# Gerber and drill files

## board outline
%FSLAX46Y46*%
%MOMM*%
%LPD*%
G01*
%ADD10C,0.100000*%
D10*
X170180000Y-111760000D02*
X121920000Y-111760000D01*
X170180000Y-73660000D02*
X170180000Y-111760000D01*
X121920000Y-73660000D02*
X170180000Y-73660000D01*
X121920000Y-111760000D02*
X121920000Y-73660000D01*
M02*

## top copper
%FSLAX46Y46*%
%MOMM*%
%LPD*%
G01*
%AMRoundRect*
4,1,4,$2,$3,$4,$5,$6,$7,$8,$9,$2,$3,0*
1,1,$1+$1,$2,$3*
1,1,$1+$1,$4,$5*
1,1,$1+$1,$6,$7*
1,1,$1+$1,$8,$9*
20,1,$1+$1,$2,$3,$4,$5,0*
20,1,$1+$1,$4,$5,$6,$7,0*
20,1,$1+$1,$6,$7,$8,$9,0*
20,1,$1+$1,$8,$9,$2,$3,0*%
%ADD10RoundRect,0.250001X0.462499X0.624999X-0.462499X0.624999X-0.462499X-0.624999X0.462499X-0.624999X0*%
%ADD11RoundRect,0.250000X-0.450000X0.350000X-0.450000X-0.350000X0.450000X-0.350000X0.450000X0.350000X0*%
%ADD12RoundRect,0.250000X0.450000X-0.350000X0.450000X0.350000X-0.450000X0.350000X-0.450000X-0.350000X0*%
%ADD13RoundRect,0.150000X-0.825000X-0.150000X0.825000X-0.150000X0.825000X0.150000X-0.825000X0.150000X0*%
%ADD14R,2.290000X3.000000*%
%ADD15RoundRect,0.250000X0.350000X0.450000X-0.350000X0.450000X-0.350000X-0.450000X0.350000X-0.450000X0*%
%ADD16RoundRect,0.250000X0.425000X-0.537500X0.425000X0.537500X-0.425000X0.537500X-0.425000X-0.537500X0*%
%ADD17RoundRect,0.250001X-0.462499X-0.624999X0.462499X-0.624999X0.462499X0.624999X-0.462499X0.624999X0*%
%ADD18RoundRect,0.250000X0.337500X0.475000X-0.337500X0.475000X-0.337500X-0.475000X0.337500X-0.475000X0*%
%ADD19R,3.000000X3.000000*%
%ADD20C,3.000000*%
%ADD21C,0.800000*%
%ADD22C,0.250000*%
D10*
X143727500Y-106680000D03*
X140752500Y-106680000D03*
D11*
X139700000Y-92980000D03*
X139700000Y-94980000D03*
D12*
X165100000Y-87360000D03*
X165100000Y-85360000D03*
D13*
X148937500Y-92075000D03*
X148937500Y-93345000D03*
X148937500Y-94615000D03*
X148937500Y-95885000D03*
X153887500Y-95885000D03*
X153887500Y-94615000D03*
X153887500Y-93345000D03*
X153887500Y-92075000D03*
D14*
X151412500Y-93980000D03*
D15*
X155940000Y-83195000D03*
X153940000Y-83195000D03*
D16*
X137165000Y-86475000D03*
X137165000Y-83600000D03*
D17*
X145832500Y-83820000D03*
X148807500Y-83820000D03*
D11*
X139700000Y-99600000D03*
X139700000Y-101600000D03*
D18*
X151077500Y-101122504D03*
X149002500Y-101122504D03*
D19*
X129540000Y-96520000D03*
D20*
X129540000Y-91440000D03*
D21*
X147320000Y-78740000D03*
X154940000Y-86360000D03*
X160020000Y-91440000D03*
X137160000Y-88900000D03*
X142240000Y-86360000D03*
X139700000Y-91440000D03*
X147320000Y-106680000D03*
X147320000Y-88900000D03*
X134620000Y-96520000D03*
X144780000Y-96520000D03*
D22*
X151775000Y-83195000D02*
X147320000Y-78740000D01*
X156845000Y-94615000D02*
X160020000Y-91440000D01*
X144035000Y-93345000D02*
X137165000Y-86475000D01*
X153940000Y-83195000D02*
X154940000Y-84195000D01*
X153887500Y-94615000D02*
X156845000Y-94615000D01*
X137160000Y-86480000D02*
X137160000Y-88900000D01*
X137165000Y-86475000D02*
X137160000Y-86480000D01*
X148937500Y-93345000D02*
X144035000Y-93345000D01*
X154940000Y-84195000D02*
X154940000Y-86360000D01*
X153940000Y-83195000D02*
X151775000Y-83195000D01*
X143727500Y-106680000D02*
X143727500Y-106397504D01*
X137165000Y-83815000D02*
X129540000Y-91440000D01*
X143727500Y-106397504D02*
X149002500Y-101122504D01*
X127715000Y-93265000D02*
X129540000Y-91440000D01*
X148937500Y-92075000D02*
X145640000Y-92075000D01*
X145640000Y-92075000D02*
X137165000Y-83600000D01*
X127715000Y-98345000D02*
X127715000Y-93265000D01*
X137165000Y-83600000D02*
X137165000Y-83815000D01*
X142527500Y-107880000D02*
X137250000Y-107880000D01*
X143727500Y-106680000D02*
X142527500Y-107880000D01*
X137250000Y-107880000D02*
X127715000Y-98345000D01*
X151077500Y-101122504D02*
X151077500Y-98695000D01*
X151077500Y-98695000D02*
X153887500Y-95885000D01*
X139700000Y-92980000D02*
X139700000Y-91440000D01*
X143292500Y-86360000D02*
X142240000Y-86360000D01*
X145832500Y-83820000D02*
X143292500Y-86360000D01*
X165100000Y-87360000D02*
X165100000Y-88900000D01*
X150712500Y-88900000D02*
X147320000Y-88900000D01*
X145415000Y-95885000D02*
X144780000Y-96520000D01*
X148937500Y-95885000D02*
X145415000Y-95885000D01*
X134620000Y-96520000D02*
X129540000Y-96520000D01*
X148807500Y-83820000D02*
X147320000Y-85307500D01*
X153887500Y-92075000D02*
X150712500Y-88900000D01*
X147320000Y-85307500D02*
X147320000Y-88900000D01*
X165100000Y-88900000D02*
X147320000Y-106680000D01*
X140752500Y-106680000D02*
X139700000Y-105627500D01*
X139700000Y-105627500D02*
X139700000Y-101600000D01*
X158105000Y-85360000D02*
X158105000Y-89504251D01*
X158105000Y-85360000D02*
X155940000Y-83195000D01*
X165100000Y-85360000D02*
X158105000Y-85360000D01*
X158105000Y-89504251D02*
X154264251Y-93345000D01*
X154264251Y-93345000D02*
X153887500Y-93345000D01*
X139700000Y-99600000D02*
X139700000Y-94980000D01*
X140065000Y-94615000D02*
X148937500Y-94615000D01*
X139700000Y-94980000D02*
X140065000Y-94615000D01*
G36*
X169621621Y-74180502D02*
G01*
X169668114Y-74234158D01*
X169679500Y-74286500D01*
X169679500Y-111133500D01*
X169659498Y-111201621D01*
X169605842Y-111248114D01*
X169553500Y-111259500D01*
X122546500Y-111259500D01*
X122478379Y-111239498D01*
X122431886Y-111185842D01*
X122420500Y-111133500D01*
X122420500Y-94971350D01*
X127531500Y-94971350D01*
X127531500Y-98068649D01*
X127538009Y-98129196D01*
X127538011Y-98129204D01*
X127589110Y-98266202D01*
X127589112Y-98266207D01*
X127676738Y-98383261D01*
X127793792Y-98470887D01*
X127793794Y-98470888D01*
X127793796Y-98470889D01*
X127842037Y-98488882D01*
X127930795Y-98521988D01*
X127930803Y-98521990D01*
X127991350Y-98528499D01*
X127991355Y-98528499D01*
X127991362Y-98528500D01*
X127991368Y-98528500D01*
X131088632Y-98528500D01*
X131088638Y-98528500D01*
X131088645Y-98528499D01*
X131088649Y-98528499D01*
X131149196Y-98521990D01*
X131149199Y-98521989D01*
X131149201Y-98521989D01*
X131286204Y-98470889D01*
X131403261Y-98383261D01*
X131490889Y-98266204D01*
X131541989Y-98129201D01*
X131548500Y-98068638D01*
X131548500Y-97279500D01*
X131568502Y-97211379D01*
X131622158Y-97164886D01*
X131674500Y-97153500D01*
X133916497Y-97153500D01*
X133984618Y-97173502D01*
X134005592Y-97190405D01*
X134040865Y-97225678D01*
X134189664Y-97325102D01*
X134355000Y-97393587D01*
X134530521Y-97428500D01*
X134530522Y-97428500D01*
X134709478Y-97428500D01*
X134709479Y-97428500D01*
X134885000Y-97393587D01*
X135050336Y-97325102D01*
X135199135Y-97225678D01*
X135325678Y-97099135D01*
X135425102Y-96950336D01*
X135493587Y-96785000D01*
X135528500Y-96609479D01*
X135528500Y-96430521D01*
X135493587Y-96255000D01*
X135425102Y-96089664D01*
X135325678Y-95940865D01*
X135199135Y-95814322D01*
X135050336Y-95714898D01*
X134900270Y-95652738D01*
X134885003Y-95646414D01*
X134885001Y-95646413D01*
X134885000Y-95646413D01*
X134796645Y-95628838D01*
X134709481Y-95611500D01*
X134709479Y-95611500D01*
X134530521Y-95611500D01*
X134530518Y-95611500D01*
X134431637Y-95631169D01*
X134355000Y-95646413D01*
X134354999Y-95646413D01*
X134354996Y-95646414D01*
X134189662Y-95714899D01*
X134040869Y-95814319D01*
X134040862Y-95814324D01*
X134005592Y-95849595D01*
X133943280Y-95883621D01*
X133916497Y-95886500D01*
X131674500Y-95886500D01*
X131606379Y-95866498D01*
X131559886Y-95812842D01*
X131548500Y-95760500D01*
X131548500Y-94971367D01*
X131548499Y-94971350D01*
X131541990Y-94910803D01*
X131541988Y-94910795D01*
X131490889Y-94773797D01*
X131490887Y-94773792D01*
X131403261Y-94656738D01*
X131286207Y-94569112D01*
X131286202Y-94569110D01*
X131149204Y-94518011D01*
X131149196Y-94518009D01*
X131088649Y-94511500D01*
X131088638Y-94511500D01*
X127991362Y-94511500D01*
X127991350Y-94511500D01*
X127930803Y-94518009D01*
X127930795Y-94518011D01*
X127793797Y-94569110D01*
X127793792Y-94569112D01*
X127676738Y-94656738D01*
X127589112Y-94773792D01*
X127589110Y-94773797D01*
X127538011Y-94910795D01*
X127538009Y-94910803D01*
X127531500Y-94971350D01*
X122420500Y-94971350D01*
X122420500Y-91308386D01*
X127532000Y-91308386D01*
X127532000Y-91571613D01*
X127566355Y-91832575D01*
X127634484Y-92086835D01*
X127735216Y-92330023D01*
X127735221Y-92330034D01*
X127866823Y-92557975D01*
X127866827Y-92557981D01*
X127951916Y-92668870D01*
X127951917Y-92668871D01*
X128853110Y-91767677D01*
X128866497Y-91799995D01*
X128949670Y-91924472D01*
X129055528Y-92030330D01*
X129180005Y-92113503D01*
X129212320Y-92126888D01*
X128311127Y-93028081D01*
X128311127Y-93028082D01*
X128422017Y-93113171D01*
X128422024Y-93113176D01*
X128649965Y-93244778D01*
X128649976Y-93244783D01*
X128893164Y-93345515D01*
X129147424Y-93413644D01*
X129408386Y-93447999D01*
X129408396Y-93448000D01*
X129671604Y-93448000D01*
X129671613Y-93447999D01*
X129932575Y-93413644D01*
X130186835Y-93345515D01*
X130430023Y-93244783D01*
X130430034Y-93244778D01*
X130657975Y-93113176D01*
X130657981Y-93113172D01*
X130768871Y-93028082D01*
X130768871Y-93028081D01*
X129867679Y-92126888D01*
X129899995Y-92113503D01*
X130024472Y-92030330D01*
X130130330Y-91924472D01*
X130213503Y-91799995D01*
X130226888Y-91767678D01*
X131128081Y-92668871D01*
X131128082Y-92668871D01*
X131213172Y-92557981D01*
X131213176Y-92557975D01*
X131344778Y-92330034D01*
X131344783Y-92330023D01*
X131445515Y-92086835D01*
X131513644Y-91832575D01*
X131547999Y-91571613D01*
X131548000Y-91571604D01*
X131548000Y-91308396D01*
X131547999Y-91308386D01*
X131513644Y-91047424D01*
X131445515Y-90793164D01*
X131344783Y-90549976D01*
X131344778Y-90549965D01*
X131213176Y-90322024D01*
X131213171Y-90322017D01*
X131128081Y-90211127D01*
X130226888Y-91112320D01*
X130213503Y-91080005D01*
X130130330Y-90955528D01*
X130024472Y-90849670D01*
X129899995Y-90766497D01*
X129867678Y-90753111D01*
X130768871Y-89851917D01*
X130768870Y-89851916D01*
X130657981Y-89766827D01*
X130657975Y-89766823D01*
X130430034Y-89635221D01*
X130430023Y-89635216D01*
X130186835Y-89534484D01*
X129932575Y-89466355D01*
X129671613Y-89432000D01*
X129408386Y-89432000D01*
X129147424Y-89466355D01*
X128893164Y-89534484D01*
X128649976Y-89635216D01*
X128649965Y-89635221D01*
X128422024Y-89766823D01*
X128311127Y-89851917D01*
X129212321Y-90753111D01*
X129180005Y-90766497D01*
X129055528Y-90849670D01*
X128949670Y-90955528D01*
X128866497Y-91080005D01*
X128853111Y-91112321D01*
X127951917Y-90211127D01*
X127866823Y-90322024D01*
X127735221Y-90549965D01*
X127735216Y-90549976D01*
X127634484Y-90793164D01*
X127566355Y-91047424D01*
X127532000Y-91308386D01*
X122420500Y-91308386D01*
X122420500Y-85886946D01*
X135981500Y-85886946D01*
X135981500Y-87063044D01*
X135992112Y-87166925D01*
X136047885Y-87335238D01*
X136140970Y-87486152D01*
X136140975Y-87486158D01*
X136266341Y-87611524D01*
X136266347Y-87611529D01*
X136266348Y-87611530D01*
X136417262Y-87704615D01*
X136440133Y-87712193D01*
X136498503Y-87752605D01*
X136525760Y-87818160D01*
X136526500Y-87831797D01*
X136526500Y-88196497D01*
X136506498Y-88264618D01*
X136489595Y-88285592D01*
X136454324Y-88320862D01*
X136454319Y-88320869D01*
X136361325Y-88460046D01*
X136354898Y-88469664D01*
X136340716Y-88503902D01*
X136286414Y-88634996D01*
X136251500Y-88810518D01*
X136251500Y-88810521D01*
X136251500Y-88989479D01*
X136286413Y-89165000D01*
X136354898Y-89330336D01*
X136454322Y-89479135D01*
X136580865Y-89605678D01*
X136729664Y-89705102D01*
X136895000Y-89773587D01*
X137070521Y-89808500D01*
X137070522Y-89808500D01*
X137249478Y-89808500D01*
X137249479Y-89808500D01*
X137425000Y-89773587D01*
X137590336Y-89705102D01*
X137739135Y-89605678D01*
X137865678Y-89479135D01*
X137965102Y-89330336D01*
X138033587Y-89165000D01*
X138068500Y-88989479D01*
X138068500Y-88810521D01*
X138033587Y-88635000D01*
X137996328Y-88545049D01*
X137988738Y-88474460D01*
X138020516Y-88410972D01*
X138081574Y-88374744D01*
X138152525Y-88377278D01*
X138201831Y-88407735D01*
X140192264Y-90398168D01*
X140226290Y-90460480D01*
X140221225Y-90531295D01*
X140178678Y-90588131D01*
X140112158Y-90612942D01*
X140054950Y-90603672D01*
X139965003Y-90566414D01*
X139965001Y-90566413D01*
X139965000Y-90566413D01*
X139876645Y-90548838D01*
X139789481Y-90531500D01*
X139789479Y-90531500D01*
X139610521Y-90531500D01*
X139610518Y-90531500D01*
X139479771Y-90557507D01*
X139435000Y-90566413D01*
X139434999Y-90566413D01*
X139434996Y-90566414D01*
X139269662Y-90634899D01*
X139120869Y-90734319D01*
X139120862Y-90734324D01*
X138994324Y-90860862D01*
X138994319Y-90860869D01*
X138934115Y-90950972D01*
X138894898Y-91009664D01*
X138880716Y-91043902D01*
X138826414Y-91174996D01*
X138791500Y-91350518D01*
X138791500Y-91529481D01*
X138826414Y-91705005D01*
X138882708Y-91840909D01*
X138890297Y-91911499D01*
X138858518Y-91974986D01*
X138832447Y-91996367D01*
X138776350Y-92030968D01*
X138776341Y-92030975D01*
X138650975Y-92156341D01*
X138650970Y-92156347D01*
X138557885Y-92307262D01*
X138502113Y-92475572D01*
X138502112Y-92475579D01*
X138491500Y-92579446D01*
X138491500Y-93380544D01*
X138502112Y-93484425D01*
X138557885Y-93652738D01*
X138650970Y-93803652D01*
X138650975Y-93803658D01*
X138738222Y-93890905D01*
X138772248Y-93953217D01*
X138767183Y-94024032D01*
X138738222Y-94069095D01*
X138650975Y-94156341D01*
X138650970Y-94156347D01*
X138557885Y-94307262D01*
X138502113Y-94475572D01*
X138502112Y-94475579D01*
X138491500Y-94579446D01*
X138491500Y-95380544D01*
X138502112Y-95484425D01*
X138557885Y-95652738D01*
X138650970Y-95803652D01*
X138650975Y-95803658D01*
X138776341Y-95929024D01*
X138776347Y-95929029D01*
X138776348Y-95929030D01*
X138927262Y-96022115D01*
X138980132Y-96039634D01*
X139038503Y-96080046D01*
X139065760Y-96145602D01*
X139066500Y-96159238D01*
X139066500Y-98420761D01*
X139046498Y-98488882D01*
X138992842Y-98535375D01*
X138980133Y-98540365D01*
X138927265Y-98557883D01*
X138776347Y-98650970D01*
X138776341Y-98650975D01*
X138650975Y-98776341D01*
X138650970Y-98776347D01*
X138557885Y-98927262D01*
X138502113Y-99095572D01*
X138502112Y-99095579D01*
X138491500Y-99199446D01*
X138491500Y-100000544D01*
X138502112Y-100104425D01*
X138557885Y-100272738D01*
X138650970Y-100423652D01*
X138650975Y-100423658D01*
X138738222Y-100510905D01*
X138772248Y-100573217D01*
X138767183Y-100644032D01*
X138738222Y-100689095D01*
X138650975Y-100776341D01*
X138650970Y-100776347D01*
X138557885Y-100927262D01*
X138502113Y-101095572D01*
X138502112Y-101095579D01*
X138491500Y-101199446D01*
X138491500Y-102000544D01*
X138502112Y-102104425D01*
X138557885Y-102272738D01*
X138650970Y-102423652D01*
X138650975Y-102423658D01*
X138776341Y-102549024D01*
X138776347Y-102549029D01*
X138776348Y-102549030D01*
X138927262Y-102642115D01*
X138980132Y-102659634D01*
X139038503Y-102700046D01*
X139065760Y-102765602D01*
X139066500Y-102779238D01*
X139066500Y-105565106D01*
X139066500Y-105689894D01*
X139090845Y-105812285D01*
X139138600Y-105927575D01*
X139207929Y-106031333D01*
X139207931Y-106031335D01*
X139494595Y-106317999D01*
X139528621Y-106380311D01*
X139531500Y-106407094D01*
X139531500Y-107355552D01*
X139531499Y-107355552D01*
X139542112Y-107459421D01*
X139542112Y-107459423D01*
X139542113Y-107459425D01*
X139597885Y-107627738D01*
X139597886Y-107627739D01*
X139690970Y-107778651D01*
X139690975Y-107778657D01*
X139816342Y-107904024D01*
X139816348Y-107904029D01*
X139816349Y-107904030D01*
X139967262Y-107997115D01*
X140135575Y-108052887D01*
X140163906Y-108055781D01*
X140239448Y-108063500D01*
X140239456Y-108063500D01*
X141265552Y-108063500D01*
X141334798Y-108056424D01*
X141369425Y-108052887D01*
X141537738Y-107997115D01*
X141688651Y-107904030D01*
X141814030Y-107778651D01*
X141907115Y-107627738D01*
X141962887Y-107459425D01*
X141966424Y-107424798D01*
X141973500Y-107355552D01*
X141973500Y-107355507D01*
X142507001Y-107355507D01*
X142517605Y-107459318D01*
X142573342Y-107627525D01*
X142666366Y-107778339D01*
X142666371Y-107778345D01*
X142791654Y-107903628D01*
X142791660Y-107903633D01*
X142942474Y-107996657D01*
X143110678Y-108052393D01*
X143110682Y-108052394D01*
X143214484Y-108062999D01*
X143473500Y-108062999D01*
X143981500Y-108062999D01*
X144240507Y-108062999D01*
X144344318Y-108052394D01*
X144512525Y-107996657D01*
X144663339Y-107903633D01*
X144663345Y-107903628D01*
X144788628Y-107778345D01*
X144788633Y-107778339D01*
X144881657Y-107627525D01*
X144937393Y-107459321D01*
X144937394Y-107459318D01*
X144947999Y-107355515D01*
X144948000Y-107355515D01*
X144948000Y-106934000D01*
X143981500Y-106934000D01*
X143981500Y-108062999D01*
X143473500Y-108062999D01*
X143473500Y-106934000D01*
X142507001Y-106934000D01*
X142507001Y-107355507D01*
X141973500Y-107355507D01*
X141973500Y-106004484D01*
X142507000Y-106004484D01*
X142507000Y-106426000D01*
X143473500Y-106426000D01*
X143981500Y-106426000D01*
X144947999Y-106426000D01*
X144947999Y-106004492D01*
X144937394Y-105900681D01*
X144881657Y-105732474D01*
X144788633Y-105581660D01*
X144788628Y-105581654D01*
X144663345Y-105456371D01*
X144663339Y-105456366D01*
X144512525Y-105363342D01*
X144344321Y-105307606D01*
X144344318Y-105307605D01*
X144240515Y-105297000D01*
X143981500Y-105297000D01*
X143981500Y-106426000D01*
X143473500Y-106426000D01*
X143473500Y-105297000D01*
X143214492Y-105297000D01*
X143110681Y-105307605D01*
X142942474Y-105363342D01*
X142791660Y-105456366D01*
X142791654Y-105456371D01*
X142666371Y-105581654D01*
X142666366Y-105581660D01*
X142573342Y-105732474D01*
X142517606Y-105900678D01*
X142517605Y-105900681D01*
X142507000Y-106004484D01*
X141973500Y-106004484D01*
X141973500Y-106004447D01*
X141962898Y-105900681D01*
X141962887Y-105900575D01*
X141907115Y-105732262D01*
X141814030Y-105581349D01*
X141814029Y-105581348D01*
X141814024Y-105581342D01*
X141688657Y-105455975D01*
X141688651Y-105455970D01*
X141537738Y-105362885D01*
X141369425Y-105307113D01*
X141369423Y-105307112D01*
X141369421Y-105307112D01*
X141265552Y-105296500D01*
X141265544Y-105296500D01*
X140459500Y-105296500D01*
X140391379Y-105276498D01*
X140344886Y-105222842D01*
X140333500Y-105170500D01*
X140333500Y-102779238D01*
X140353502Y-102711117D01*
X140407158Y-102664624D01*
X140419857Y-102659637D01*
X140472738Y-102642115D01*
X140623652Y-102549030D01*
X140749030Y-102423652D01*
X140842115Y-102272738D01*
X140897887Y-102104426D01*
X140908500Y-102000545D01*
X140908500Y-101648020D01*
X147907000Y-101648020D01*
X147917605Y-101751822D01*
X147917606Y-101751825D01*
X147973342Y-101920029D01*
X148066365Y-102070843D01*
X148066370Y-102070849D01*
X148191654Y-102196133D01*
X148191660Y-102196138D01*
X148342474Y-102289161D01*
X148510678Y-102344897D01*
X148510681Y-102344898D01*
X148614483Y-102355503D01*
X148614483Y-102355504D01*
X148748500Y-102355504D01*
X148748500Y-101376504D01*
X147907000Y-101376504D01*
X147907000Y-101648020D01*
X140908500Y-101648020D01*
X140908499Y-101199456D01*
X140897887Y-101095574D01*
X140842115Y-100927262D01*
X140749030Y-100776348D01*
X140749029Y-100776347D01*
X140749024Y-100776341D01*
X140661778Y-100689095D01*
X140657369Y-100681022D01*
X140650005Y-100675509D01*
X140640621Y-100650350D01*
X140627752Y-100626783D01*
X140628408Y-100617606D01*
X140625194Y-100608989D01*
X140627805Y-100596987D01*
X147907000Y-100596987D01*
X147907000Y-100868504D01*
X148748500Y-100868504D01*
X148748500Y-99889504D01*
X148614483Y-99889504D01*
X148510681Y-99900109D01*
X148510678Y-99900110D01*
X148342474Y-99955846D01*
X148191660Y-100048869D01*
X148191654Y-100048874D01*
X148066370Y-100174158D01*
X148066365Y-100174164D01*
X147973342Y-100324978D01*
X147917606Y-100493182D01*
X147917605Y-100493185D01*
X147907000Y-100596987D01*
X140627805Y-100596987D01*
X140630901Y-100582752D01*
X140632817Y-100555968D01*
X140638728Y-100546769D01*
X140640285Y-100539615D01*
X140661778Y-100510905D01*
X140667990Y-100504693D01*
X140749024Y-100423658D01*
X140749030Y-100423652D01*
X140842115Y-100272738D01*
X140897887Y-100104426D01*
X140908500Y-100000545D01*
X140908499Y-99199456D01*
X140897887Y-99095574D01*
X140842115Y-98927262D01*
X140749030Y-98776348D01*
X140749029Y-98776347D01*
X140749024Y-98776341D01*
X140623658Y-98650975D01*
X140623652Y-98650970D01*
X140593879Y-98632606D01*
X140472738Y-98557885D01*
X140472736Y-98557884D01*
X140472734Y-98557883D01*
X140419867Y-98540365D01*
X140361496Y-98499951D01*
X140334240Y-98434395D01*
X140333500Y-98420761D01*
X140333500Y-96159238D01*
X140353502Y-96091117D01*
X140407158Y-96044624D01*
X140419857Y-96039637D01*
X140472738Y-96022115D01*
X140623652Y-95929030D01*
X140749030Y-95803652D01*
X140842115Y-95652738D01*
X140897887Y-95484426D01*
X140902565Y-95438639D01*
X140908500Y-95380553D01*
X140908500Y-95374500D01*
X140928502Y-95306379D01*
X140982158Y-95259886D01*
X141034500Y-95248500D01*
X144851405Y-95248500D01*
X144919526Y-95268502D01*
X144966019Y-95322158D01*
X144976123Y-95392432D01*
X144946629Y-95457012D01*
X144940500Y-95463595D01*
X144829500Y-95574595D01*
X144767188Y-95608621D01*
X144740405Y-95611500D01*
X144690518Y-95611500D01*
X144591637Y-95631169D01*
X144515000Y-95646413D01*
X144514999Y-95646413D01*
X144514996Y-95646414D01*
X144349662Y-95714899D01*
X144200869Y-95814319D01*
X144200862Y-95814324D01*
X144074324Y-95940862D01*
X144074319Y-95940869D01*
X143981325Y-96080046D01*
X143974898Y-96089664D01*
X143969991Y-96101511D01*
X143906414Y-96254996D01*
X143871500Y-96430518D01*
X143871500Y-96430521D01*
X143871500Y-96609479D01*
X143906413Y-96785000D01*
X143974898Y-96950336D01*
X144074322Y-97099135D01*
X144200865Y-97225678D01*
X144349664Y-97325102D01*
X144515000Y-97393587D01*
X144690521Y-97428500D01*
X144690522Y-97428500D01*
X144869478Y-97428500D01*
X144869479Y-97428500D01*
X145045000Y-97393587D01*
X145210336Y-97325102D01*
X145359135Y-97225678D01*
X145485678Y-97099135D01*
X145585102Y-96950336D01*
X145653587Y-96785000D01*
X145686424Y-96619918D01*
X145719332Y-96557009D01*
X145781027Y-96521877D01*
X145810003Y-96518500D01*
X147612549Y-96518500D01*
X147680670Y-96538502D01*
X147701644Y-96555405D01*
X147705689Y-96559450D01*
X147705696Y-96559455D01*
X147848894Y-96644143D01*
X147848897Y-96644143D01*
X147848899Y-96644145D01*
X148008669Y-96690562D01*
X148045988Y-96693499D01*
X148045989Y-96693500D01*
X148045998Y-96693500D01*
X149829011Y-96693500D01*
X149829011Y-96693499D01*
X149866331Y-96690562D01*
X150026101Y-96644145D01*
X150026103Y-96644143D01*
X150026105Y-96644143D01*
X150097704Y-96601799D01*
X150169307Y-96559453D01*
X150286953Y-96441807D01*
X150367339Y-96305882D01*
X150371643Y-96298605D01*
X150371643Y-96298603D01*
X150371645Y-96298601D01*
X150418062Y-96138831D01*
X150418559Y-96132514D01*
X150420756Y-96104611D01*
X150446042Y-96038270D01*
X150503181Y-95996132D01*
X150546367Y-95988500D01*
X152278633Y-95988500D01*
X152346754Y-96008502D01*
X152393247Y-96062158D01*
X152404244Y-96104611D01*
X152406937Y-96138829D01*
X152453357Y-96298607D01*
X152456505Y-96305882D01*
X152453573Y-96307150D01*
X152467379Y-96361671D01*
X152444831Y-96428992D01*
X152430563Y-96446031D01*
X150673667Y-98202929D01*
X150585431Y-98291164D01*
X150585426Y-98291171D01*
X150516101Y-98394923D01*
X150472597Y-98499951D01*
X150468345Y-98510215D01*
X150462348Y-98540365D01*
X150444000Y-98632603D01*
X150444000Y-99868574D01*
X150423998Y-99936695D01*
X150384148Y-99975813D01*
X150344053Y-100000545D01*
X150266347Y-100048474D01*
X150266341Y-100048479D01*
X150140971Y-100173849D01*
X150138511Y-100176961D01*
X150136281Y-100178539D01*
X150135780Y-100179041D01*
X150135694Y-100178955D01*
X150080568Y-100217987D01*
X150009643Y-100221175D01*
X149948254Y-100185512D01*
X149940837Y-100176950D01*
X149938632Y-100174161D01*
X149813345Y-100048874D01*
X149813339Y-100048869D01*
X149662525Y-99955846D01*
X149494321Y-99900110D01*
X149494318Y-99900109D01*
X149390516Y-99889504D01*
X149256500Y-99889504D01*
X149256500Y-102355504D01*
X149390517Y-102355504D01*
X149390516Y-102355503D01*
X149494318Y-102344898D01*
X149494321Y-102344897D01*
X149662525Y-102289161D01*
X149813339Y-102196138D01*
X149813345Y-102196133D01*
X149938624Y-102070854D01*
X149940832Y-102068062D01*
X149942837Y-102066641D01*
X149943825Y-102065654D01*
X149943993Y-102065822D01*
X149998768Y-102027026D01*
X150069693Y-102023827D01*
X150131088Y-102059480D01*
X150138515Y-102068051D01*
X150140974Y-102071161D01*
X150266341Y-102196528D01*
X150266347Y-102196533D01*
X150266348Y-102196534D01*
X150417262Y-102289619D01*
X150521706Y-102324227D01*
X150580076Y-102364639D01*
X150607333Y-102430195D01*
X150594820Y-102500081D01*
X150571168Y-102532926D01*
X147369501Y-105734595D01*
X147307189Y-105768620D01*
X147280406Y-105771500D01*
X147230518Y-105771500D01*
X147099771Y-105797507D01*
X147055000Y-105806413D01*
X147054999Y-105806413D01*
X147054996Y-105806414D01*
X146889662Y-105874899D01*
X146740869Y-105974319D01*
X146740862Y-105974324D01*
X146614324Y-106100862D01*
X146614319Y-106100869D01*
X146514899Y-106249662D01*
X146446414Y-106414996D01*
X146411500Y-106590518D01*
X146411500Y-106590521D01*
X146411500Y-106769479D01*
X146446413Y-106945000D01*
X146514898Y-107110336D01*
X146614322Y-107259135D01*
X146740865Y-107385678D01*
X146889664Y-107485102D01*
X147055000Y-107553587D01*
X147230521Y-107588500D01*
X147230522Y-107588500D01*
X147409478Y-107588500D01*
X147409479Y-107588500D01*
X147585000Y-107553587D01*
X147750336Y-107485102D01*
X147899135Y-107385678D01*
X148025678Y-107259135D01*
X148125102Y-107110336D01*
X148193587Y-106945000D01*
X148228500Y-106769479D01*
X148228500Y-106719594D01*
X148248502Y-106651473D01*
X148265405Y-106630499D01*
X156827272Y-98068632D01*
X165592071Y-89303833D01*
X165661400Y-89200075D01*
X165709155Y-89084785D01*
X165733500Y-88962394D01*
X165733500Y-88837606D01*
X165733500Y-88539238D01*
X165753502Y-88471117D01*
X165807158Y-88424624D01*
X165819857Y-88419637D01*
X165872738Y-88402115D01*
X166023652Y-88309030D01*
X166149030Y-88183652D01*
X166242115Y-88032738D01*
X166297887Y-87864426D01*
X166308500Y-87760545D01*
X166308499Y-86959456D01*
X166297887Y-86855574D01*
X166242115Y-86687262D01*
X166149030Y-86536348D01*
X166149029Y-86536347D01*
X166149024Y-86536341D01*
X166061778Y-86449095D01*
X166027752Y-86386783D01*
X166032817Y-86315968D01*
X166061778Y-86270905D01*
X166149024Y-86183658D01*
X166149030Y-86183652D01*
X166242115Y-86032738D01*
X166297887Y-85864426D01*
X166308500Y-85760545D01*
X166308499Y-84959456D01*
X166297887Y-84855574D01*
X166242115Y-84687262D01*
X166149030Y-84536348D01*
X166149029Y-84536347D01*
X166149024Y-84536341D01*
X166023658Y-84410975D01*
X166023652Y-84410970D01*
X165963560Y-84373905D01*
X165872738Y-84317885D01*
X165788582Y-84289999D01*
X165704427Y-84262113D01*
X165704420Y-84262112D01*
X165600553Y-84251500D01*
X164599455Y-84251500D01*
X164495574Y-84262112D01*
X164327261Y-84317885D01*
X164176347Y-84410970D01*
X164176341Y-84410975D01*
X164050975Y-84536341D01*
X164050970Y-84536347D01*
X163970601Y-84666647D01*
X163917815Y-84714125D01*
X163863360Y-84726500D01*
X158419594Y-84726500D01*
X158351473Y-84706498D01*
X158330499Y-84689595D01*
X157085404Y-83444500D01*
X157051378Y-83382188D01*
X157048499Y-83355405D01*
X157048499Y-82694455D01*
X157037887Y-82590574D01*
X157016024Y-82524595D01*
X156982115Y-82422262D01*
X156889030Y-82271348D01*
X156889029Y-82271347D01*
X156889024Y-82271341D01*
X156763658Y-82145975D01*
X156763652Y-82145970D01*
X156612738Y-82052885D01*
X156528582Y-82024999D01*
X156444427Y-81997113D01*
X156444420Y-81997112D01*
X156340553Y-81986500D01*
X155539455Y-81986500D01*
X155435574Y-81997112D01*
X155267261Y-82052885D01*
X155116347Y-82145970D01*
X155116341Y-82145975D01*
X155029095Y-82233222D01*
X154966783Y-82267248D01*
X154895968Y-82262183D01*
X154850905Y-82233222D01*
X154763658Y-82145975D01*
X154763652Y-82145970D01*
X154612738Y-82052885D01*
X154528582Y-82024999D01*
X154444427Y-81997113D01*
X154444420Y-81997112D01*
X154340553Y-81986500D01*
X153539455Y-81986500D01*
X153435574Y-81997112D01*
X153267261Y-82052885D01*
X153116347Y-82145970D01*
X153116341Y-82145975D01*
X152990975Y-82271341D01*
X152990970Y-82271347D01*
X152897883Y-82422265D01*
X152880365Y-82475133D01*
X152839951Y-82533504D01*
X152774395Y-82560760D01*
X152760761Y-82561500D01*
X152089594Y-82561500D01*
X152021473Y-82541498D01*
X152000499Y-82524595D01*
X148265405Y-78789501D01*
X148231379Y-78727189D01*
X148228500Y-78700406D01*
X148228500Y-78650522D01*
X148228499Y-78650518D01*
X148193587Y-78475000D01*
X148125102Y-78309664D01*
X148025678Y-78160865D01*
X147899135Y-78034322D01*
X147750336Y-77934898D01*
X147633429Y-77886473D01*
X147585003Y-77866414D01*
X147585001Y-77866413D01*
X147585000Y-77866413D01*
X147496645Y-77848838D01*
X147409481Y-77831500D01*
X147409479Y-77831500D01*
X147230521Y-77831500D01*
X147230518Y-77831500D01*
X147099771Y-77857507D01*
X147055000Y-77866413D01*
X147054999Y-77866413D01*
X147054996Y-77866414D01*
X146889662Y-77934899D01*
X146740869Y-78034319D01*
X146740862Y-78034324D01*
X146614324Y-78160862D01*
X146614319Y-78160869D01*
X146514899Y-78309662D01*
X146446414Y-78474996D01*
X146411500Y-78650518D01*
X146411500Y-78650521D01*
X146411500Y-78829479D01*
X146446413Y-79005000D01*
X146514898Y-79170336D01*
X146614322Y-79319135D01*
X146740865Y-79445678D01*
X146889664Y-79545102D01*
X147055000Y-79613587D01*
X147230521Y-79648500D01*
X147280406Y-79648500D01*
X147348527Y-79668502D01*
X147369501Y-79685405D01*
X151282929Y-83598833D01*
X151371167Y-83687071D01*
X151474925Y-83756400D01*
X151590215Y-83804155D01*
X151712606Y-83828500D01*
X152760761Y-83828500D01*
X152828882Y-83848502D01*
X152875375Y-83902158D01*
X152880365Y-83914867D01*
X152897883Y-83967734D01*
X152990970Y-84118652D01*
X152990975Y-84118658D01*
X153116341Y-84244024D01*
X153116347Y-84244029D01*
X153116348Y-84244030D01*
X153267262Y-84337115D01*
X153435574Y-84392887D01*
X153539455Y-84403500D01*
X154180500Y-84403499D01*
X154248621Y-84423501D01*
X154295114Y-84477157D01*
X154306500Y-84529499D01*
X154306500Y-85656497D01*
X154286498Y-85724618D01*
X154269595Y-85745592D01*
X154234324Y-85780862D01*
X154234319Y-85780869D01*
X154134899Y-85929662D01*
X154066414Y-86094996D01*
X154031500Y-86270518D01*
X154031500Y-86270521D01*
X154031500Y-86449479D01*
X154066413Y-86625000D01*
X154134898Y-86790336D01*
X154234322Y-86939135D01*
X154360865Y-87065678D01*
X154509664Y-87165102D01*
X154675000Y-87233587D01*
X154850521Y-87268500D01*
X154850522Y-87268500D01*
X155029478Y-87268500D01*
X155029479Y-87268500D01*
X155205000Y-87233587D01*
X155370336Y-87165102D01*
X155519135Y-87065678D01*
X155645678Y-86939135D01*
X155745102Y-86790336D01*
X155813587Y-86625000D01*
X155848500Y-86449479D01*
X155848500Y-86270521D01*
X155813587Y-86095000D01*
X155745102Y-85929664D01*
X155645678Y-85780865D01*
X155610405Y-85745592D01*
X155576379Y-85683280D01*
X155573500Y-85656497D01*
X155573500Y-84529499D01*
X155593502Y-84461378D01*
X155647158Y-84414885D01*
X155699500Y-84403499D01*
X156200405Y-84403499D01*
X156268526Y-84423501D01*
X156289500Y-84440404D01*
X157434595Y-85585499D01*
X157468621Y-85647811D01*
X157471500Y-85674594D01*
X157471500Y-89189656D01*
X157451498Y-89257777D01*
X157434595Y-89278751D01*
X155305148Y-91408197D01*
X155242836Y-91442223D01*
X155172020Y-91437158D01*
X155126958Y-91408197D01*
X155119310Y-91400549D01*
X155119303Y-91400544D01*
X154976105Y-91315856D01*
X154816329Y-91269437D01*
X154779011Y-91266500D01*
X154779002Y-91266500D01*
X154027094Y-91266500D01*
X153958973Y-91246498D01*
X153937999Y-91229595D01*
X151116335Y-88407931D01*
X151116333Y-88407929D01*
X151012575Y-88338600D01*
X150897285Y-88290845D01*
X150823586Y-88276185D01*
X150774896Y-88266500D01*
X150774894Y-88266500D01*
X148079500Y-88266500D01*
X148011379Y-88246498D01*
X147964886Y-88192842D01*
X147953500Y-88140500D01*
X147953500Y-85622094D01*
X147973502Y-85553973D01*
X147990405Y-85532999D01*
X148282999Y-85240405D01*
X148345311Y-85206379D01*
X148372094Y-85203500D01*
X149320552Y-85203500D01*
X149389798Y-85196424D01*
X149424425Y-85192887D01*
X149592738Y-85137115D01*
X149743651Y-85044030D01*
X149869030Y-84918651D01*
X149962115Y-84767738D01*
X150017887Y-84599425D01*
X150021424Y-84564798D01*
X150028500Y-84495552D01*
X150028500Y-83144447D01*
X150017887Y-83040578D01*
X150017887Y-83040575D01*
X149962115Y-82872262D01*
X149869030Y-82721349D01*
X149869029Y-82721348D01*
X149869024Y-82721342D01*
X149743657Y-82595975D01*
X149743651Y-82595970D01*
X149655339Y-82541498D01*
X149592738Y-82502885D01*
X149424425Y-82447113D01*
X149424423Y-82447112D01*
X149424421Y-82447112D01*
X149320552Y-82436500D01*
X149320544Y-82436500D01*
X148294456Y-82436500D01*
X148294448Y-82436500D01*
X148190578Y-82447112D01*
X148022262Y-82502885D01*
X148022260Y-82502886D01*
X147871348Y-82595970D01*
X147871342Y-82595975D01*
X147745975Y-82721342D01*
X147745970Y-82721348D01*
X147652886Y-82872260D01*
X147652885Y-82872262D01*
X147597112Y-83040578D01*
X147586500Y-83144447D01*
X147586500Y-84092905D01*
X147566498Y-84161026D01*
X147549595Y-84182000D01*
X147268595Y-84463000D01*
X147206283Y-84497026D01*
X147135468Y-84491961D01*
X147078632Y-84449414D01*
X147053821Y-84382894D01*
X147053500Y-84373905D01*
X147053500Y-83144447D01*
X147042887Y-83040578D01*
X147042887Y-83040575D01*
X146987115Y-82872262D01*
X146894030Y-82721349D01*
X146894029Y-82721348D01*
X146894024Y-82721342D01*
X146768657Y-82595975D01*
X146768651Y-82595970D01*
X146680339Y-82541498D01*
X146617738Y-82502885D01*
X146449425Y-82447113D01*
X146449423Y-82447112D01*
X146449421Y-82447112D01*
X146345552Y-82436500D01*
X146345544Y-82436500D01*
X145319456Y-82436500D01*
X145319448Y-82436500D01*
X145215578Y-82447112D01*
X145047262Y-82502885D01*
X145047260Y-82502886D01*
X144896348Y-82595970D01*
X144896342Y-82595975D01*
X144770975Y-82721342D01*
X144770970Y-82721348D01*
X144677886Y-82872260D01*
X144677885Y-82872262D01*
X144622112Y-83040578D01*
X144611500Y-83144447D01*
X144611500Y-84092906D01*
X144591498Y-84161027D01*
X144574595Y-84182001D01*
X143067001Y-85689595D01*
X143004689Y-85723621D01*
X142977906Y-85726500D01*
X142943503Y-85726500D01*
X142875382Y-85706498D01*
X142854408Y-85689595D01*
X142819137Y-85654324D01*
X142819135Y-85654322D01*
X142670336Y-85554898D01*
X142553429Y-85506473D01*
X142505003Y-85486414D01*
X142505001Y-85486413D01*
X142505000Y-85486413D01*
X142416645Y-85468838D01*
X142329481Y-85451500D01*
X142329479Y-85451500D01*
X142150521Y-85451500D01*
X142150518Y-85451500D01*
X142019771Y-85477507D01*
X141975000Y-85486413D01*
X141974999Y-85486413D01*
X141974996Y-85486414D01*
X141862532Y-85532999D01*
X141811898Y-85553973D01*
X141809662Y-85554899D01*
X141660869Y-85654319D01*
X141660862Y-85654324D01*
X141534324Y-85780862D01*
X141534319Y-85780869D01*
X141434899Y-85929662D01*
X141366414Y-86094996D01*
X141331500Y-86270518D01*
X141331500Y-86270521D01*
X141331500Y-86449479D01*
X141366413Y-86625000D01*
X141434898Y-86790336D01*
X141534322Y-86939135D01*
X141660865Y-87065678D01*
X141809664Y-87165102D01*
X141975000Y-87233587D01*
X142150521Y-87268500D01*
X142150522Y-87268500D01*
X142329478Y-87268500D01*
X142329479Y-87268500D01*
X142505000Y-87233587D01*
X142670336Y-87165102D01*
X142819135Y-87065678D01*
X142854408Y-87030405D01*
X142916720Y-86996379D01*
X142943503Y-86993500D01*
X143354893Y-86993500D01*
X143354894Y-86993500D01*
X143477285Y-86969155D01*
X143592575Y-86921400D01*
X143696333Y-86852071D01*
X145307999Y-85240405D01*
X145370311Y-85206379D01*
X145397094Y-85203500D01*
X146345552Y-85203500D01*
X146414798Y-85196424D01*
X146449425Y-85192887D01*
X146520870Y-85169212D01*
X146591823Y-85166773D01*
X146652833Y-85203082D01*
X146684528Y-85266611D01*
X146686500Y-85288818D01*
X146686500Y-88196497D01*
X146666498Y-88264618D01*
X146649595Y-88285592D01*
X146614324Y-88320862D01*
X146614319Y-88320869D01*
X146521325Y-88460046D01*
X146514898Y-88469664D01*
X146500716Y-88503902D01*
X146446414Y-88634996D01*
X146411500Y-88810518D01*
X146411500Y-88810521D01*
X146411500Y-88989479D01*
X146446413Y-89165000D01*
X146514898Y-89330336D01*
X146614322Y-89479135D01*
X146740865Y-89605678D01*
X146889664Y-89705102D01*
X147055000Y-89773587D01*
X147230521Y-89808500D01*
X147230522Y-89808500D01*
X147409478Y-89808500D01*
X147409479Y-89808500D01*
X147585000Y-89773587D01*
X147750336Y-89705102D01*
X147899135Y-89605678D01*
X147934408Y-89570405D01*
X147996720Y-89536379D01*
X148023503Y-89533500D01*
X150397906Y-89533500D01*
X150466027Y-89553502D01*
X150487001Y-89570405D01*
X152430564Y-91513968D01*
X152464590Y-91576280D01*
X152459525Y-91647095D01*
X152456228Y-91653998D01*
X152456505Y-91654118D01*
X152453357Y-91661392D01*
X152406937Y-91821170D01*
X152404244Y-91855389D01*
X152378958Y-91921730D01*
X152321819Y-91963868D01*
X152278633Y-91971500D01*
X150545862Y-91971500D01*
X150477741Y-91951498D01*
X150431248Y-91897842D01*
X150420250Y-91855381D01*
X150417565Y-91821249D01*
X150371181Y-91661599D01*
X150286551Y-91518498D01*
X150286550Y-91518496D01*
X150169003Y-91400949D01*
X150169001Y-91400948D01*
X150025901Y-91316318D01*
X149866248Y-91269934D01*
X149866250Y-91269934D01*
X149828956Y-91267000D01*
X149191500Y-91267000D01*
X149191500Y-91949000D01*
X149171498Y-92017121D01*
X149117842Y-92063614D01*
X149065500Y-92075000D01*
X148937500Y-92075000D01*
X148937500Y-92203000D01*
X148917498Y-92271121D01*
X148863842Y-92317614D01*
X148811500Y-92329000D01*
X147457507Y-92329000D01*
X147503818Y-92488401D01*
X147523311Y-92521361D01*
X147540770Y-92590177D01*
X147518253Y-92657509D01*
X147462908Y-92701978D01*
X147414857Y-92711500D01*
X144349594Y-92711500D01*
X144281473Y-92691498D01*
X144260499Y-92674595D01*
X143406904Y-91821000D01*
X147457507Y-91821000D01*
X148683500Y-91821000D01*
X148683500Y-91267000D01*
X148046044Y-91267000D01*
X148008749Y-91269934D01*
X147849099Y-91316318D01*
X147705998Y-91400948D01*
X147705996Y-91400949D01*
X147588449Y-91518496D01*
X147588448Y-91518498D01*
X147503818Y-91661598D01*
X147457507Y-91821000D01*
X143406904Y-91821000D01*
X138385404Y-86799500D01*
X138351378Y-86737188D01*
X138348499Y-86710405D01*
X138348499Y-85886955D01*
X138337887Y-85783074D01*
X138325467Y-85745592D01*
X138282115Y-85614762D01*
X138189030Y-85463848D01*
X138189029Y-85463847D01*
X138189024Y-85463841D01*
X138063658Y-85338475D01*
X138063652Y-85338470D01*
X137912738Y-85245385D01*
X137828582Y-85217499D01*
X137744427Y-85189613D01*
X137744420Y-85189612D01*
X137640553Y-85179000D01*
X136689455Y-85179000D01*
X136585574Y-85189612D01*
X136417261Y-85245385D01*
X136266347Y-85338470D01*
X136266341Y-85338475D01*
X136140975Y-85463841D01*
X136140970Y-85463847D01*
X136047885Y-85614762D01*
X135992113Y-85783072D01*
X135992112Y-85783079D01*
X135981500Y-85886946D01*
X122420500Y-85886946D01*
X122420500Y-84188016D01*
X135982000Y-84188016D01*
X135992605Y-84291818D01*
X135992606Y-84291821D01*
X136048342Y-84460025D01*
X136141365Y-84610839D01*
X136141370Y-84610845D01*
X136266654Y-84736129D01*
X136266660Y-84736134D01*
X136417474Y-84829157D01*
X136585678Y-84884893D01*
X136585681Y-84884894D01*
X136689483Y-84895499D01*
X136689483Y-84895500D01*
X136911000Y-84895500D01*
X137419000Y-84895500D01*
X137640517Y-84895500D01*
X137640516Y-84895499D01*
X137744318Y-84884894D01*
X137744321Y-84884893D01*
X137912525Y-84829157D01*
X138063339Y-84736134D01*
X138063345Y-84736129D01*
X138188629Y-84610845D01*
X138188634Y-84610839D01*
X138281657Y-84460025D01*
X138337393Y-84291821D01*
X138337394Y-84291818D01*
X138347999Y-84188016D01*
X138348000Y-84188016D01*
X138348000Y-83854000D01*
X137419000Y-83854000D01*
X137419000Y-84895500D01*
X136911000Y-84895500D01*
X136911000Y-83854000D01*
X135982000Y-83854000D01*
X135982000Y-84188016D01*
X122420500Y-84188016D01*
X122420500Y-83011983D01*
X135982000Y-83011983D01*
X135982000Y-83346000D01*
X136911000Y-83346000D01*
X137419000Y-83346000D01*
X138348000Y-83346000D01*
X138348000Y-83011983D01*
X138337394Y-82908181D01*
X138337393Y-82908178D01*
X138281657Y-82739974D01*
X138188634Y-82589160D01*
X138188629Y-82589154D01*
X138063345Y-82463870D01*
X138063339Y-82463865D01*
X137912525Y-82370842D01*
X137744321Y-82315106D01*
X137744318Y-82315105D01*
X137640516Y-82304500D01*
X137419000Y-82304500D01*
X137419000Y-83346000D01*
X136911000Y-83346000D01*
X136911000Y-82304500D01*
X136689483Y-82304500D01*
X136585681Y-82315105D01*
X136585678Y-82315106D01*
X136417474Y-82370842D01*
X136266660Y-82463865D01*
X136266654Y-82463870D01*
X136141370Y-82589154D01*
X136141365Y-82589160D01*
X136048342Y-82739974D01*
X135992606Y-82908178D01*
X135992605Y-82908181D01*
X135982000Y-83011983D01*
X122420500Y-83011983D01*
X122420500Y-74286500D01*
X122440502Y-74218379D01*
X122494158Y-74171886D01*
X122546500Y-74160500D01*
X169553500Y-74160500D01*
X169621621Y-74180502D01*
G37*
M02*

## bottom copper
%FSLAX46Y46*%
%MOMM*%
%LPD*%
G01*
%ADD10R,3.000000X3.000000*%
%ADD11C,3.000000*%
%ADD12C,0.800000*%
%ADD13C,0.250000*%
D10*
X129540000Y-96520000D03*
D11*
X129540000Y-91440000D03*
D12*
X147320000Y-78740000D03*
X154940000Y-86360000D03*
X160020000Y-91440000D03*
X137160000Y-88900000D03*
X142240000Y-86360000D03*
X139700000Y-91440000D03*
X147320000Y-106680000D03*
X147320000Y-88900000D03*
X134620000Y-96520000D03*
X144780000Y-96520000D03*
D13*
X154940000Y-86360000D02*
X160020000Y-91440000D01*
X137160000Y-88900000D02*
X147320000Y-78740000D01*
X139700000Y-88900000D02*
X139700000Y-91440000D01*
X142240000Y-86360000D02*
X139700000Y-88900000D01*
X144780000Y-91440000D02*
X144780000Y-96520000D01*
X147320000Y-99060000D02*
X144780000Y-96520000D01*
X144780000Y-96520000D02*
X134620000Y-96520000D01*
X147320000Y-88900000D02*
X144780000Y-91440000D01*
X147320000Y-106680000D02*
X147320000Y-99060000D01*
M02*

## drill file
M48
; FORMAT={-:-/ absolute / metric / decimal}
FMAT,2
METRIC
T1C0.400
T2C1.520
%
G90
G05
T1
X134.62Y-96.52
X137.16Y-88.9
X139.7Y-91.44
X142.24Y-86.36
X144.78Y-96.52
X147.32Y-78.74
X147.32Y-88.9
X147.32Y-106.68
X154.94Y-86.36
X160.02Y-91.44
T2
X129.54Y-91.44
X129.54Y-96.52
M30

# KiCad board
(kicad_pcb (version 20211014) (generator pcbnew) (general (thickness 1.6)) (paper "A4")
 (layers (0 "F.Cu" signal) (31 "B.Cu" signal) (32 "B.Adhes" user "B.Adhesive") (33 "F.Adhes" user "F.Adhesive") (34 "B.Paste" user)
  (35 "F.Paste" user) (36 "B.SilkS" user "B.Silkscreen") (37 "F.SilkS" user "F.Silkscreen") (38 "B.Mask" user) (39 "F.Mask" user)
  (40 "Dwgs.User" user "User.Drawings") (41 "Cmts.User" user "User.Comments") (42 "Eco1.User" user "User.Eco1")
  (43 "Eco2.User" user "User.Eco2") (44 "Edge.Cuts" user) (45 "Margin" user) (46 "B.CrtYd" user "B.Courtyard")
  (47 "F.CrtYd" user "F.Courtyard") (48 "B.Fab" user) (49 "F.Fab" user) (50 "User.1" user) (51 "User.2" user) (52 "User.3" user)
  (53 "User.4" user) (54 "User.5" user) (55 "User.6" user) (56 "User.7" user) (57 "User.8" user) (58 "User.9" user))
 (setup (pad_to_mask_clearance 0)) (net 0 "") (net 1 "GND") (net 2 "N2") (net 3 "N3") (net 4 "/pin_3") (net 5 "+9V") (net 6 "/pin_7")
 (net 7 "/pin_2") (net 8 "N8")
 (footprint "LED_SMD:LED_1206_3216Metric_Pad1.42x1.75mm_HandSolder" (layer "F.Cu") (at 142.24 106.68 180)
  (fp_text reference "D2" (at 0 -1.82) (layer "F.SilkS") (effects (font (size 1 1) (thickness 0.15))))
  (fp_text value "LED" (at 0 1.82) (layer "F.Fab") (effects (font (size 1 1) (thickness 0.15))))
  (pad "1" smd roundrect (at -1.4875 0 180) (size 1.425 1.75) (layers "F.Cu" "F.Paste" "F.Mask") (roundrect_rratio 0.1754392982)
   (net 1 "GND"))
  (pad "2" smd roundrect (at 1.4875 0 180) (size 1.425 1.75) (layers "F.Cu" "F.Paste" "F.Mask") (roundrect_rratio 0.1754392982) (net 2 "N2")))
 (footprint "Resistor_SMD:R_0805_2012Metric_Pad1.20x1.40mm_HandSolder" (layer "F.Cu") (at 139.7 93.98 -90)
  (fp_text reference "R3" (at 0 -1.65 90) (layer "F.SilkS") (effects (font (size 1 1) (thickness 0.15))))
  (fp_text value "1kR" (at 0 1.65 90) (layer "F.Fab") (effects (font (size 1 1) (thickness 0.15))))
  (pad "1" smd roundrect (at -1 0 270) (size 1.2 1.4) (layers "F.Cu" "F.Paste" "F.Mask") (roundrect_rratio 0.2083333333) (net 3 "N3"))
  (pad "2" smd roundrect (at 1 0 270) (size 1.2 1.4) (layers "F.Cu" "F.Paste" "F.Mask") (roundrect_rratio 0.2083333333) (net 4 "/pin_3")))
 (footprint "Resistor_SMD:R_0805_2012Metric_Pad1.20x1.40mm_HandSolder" (layer "F.Cu") (at 165.1 86.36 90)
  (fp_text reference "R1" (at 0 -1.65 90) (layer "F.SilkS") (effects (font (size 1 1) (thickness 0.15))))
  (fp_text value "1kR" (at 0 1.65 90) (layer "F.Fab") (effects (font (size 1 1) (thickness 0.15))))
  (pad "1" smd roundrect (at -1 0 90) (size 1.2 1.4) (layers "F.Cu" "F.Paste" "F.Mask") (roundrect_rratio 0.2083333333) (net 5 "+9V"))
  (pad "2" smd roundrect (at 1 0 90) (size 1.2 1.4) (layers "F.Cu" "F.Paste" "F.Mask") (roundrect_rratio 0.2083333333) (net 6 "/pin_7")))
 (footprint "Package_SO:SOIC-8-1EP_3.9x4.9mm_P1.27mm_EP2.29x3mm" (layer "F.Cu") (at 151.4125 93.98)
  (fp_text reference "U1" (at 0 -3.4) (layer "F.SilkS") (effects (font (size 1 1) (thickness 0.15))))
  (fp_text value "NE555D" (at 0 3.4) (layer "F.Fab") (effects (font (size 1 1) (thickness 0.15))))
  (pad "" smd roundrect (at 0.57 0.75) (size 0.92 1.21) (layers "F.Paste") (roundrect_rratio 0.25))
  (pad "" smd roundrect (at 0.57 -0.75) (size 0.92 1.21) (layers "F.Paste") (roundrect_rratio 0.25))
  (pad "" smd roundrect (at -0.57 -0.75) (size 0.92 1.21) (layers "F.Paste") (roundrect_rratio 0.25))
  (pad "" smd roundrect (at -0.57 0.75) (size 0.92 1.21) (layers "F.Paste") (roundrect_rratio 0.25))
  (pad "1" smd roundrect (at -2.475 -1.905) (size 1.95 0.6) (layers "F.Cu" "F.Paste" "F.Mask") (roundrect_rratio 0.25) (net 1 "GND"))
  (pad "2" smd roundrect (at -2.475 -0.635) (size 1.95 0.6) (layers "F.Cu" "F.Paste" "F.Mask") (roundrect_rratio 0.25) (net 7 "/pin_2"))
  (pad "3" smd roundrect (at -2.475 0.635) (size 1.95 0.6) (layers "F.Cu" "F.Paste" "F.Mask") (roundrect_rratio 0.25) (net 4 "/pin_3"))
  (pad "4" smd roundrect (at -2.475 1.905) (size 1.95 0.6) (layers "F.Cu" "F.Paste" "F.Mask") (roundrect_rratio 0.25) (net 5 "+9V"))
  (pad "5" smd roundrect (at 2.475 1.905) (size 1.95 0.6) (layers "F.Cu" "F.Paste" "F.Mask") (roundrect_rratio 0.25) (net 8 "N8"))
  (pad "6" smd roundrect (at 2.475 0.635) (size 1.95 0.6) (layers "F.Cu" "F.Paste" "F.Mask") (roundrect_rratio 0.25) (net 7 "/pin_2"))
  (pad "7" smd roundrect (at 2.475 -0.635) (size 1.95 0.6) (layers "F.Cu" "F.Paste" "F.Mask") (roundrect_rratio 0.25) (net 6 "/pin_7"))
  (pad "8" smd roundrect (at 2.475 -1.905) (size 1.95 0.6) (layers "F.Cu" "F.Paste" "F.Mask") (roundrect_rratio 0.25) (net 5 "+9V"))
  (pad "9" smd rect (at 0 0) (size 2.29 3) (layers "F.Cu" "F.Mask")))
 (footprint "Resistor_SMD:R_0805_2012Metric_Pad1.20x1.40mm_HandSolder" (layer "F.Cu") (at 154.94 83.195 180)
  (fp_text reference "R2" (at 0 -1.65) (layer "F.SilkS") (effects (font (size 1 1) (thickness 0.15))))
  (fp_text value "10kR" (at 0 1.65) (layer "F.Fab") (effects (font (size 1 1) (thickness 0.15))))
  (pad "1" smd roundrect (at -1 0 180) (size 1.2 1.4) (layers "F.Cu" "F.Paste" "F.Mask") (roundrect_rratio 0.2083333333) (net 6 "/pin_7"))
  (pad "2" smd roundrect (at 1 0 180) (size 1.2 1.4) (layers "F.Cu" "F.Paste" "F.Mask") (roundrect_rratio 0.2083333333) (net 7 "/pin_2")))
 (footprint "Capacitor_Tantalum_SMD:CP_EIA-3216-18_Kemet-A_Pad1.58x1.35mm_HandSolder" (layer "F.Cu") (at 137.165 85.0375 90)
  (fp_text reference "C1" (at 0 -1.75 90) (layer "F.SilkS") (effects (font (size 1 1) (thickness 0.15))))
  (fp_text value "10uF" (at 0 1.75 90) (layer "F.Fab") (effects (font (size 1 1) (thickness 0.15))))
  (pad "1" smd roundrect (at -1.4375 0 90) (size 1.575 1.35) (layers "F.Cu" "F.Paste" "F.Mask") (roundrect_rratio 0.1851851852)
   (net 7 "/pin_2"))
  (pad "2" smd roundrect (at 1.4375 0 90) (size 1.575 1.35) (layers "F.Cu" "F.Paste" "F.Mask") (roundrect_rratio 0.1851851852) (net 1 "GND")))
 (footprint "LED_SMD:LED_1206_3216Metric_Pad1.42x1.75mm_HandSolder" (layer "F.Cu") (at 147.32 83.82)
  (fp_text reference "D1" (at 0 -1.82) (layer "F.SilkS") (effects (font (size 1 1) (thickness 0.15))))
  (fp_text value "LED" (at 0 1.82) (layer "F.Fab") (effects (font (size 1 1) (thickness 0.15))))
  (pad "1" smd roundrect (at -1.4875 0) (size 1.425 1.75) (layers "F.Cu" "F.Paste" "F.Mask") (roundrect_rratio 0.1754392982) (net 3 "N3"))
  (pad "2" smd roundrect (at 1.4875 0) (size 1.425 1.75) (layers "F.Cu" "F.Paste" "F.Mask") (roundrect_rratio 0.1754392982) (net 5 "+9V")))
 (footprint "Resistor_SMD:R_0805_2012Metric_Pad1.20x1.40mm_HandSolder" (layer "F.Cu") (at 139.7 100.6 -90)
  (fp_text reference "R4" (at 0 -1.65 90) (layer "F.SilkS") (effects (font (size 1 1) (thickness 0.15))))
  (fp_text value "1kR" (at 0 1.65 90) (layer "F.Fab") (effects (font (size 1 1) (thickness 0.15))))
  (pad "1" smd roundrect (at -1 0 270) (size 1.2 1.4) (layers "F.Cu" "F.Paste" "F.Mask") (roundrect_rratio 0.2083333333) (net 4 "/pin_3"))
  (pad "2" smd roundrect (at 1 0 270) (size 1.2 1.4) (layers "F.Cu" "F.Paste" "F.Mask") (roundrect_rratio 0.2083333333) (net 2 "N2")))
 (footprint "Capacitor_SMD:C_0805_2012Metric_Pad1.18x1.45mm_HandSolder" (layer "F.Cu") (at 150.04 101.122504 180)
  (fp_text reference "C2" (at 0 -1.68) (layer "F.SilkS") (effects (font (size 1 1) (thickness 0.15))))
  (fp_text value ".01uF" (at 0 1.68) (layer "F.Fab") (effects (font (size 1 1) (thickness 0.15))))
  (pad "1" smd roundrect (at -1.0375 0 180) (size 1.175 1.45) (layers "F.Cu" "F.Paste" "F.Mask") (roundrect_rratio 0.2127659574)
   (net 8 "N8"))
  (pad "2" smd roundrect (at 1.0375 0 180) (size 1.175 1.45) (layers "F.Cu" "F.Paste" "F.Mask") (roundrect_rratio 0.2127659574)
   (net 1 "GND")))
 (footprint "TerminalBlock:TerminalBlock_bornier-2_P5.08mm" (layer "B.Cu") (at 129.54 96.52 90)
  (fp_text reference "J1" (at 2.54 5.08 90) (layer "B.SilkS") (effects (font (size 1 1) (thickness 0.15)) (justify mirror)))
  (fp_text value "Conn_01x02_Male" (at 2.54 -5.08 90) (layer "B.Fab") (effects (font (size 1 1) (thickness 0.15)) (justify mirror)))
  (pad "1" thru_hole rect (at 0 0 90) (size 3 3) (drill 1.52) (layers *.Cu *.Mask) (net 5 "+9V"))
  (pad "2" thru_hole circle (at 5.08 0 90) (size 3 3) (drill 1.52) (layers *.Cu *.Mask) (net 1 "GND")))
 (gr_line (start 170.18 111.76) (end 121.92 111.76) (layer "Edge.Cuts") (width 0.1))
 (gr_line (start 170.18 73.66) (end 170.18 111.76) (layer "Edge.Cuts") (width 0.1))
 (gr_line (start 121.92 73.66) (end 170.18 73.66) (layer "Edge.Cuts") (width 0.1))
 (gr_line (start 121.92 111.76) (end 121.92 73.66) (layer "Edge.Cuts") (width 0.1))
 (segment (start 151.775 83.195) (end 147.32 78.74) (width 0.25) (layer "F.Cu") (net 7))
 (segment (start 156.845 94.615) (end 160.02 91.44) (width 0.25) (layer "F.Cu") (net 7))
 (segment (start 144.035 93.345) (end 137.165 86.475) (width 0.25) (layer "F.Cu") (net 7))
 (segment (start 153.94 83.195) (end 154.94 84.195) (width 0.25) (layer "F.Cu") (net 7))
 (segment (start 153.8875 94.615) (end 156.845 94.615) (width 0.25) (layer "F.Cu") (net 7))
 (segment (start 137.16 86.48) (end 137.16 88.9) (width 0.25) (layer "F.Cu") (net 7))
 (segment (start 137.165 86.475) (end 137.16 86.48) (width 0.25) (layer "F.Cu") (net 7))
 (segment (start 148.9375 93.345) (end 144.035 93.345) (width 0.25) (layer "F.Cu") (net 7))
 (segment (start 154.94 84.195) (end 154.94 86.36) (width 0.25) (layer "F.Cu") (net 7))
 (segment (start 153.94 83.195) (end 151.775 83.195) (width 0.25) (layer "F.Cu") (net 7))
 (via (at 147.32 78.74) (size 0.8) (drill 0.4) (layers "F.Cu" "B.Cu") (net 7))
 (via (at 154.94 86.36) (size 0.8) (drill 0.4) (layers "F.Cu" "B.Cu") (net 7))
 (via (at 160.02 91.44) (size 0.8) (drill 0.4) (layers "F.Cu" "B.Cu") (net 7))
 (via (at 137.16 88.9) (size 0.8) (drill 0.4) (layers "F.Cu" "B.Cu") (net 7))
 (segment (start 154.94 86.36) (end 160.02 91.44) (width 0.25) (layer "B.Cu") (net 7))
 (segment (start 137.16 88.9) (end 147.32 78.74) (width 0.25) (layer "B.Cu") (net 7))
 (segment (start 143.7275 106.68) (end 143.7275 106.397504) (width 0.25) (layer "F.Cu") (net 1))
 (segment (start 137.165 83.815) (end 129.54 91.44) (width 0.25) (layer "F.Cu") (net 1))
 (segment (start 143.7275 106.397504) (end 149.0025 101.122504) (width 0.25) (layer "F.Cu") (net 1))
 (segment (start 127.715 93.265) (end 129.54 91.44) (width 0.25) (layer "F.Cu") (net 1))
 (segment (start 148.9375 92.075) (end 145.64 92.075) (width 0.25) (layer "F.Cu") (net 1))
 (segment (start 145.64 92.075) (end 137.165 83.6) (width 0.25) (layer "F.Cu") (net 1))
 (segment (start 127.715 98.345) (end 127.715 93.265) (width 0.25) (layer "F.Cu") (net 1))
 (segment (start 137.165 83.6) (end 137.165 83.815) (width 0.25) (layer "F.Cu") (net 1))
 (segment (start 142.5275 107.88) (end 137.25 107.88) (width 0.25) (layer "F.Cu") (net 1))
 (segment (start 143.7275 106.68) (end 142.5275 107.88) (width 0.25) (layer "F.Cu") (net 1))
 (segment (start 137.25 107.88) (end 127.715 98.345) (width 0.25) (layer "F.Cu") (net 1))
 (segment (start 151.0775 101.122504) (end 151.0775 98.695) (width 0.25) (layer "F.Cu") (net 8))
 (segment (start 151.0775 98.695) (end 153.8875 95.885) (width 0.25) (layer "F.Cu") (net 8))
 (segment (start 139.7 92.98) (end 139.7 91.44) (width 0.25) (layer "F.Cu") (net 3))
 (segment (start 143.2925 86.36) (end 142.24 86.36) (width 0.25) (layer "F.Cu") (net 3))
 (segment (start 145.8325 83.82) (end 143.2925 86.36) (width 0.25) (layer "F.Cu") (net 3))
 (via (at 142.24 86.36) (size 0.8) (drill 0.4) (layers "F.Cu" "B.Cu") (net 3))
 (via (at 139.7 91.44) (size 0.8) (drill 0.4) (layers "F.Cu" "B.Cu") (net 3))
 (segment (start 139.7 88.9) (end 139.7 91.44) (width 0.25) (layer "B.Cu") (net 3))
 (segment (start 142.24 86.36) (end 139.7 88.9) (width 0.25) (layer "B.Cu") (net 3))
 (segment (start 165.1 87.36) (end 165.1 88.9) (width 0.25) (layer "F.Cu") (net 5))
 (segment (start 150.7125 88.9) (end 147.32 88.9) (width 0.25) (layer "F.Cu") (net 5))
 (segment (start 145.415 95.885) (end 144.78 96.52) (width 0.25) (layer "F.Cu") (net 5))
 (segment (start 148.9375 95.885) (end 145.415 95.885) (width 0.25) (layer "F.Cu") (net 5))
 (segment (start 134.62 96.52) (end 129.54 96.52) (width 0.25) (layer "F.Cu") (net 5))
 (segment (start 148.8075 83.82) (end 147.32 85.3075) (width 0.25) (layer "F.Cu") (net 5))
 (segment (start 153.8875 92.075) (end 150.7125 88.9) (width 0.25) (layer "F.Cu") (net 5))
 (segment (start 147.32 85.3075) (end 147.32 88.9) (width 0.25) (layer "F.Cu") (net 5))
 (segment (start 165.1 88.9) (end 147.32 106.68) (width 0.25) (layer "F.Cu") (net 5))
 (via (at 147.32 106.68) (size 0.8) (drill 0.4) (layers "F.Cu" "B.Cu") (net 5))
 (via (at 147.32 88.9) (size 0.8) (drill 0.4) (layers "F.Cu" "B.Cu") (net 5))
 (via (at 134.62 96.52) (size 0.8) (drill 0.4) (layers "F.Cu" "B.Cu") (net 5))
 (via (at 144.78 96.52) (size 0.8) (drill 0.4) (layers "F.Cu" "B.Cu") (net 5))
 (segment (start 144.78 91.44) (end 144.78 96.52) (width 0.25) (layer "B.Cu") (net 5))
 (segment (start 147.32 99.06) (end 144.78 96.52) (width 0.25) (layer "B.Cu") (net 5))
 (segment (start 144.78 96.52) (end 134.62 96.52) (width 0.25) (layer "B.Cu") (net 5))
 (segment (start 147.32 88.9) (end 144.78 91.44) (width 0.25) (layer "B.Cu") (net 5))
 (segment (start 147.32 106.68) (end 147.32 99.06) (width 0.25) (layer "B.Cu") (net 5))
 (segment (start 140.7525 106.68) (end 139.7 105.6275) (width 0.25) (layer "F.Cu") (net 2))
 (segment (start 139.7 105.6275) (end 139.7 101.6) (width 0.25) (layer "F.Cu") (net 2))
 (segment (start 158.105 85.36) (end 158.105 89.504251) (width 0.25) (layer "F.Cu") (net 6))
 (segment (start 158.105 85.36) (end 155.94 83.195) (width 0.25) (layer "F.Cu") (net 6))
 (segment (start 165.1 85.36) (end 158.105 85.36) (width 0.25) (layer "F.Cu") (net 6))
 (segment (start 158.105 89.504251) (end 154.264251 93.345) (width 0.25) (layer "F.Cu") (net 6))
 (segment (start 154.264251 93.345) (end 153.8875 93.345) (width 0.25) (layer "F.Cu") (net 6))
 (segment (start 139.7 99.6) (end 139.7 94.98) (width 0.25) (layer "F.Cu") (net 4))
 (segment (start 140.065 94.615) (end 148.9375 94.615) (width 0.25) (layer "F.Cu") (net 4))
 (segment (start 139.7 94.98) (end 140.065 94.615) (width 0.25) (layer "F.Cu") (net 4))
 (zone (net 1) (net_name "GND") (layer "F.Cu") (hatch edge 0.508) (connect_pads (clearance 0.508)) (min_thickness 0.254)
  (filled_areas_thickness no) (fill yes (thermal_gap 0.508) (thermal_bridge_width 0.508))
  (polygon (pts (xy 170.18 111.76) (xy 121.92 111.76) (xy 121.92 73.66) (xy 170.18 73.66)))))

